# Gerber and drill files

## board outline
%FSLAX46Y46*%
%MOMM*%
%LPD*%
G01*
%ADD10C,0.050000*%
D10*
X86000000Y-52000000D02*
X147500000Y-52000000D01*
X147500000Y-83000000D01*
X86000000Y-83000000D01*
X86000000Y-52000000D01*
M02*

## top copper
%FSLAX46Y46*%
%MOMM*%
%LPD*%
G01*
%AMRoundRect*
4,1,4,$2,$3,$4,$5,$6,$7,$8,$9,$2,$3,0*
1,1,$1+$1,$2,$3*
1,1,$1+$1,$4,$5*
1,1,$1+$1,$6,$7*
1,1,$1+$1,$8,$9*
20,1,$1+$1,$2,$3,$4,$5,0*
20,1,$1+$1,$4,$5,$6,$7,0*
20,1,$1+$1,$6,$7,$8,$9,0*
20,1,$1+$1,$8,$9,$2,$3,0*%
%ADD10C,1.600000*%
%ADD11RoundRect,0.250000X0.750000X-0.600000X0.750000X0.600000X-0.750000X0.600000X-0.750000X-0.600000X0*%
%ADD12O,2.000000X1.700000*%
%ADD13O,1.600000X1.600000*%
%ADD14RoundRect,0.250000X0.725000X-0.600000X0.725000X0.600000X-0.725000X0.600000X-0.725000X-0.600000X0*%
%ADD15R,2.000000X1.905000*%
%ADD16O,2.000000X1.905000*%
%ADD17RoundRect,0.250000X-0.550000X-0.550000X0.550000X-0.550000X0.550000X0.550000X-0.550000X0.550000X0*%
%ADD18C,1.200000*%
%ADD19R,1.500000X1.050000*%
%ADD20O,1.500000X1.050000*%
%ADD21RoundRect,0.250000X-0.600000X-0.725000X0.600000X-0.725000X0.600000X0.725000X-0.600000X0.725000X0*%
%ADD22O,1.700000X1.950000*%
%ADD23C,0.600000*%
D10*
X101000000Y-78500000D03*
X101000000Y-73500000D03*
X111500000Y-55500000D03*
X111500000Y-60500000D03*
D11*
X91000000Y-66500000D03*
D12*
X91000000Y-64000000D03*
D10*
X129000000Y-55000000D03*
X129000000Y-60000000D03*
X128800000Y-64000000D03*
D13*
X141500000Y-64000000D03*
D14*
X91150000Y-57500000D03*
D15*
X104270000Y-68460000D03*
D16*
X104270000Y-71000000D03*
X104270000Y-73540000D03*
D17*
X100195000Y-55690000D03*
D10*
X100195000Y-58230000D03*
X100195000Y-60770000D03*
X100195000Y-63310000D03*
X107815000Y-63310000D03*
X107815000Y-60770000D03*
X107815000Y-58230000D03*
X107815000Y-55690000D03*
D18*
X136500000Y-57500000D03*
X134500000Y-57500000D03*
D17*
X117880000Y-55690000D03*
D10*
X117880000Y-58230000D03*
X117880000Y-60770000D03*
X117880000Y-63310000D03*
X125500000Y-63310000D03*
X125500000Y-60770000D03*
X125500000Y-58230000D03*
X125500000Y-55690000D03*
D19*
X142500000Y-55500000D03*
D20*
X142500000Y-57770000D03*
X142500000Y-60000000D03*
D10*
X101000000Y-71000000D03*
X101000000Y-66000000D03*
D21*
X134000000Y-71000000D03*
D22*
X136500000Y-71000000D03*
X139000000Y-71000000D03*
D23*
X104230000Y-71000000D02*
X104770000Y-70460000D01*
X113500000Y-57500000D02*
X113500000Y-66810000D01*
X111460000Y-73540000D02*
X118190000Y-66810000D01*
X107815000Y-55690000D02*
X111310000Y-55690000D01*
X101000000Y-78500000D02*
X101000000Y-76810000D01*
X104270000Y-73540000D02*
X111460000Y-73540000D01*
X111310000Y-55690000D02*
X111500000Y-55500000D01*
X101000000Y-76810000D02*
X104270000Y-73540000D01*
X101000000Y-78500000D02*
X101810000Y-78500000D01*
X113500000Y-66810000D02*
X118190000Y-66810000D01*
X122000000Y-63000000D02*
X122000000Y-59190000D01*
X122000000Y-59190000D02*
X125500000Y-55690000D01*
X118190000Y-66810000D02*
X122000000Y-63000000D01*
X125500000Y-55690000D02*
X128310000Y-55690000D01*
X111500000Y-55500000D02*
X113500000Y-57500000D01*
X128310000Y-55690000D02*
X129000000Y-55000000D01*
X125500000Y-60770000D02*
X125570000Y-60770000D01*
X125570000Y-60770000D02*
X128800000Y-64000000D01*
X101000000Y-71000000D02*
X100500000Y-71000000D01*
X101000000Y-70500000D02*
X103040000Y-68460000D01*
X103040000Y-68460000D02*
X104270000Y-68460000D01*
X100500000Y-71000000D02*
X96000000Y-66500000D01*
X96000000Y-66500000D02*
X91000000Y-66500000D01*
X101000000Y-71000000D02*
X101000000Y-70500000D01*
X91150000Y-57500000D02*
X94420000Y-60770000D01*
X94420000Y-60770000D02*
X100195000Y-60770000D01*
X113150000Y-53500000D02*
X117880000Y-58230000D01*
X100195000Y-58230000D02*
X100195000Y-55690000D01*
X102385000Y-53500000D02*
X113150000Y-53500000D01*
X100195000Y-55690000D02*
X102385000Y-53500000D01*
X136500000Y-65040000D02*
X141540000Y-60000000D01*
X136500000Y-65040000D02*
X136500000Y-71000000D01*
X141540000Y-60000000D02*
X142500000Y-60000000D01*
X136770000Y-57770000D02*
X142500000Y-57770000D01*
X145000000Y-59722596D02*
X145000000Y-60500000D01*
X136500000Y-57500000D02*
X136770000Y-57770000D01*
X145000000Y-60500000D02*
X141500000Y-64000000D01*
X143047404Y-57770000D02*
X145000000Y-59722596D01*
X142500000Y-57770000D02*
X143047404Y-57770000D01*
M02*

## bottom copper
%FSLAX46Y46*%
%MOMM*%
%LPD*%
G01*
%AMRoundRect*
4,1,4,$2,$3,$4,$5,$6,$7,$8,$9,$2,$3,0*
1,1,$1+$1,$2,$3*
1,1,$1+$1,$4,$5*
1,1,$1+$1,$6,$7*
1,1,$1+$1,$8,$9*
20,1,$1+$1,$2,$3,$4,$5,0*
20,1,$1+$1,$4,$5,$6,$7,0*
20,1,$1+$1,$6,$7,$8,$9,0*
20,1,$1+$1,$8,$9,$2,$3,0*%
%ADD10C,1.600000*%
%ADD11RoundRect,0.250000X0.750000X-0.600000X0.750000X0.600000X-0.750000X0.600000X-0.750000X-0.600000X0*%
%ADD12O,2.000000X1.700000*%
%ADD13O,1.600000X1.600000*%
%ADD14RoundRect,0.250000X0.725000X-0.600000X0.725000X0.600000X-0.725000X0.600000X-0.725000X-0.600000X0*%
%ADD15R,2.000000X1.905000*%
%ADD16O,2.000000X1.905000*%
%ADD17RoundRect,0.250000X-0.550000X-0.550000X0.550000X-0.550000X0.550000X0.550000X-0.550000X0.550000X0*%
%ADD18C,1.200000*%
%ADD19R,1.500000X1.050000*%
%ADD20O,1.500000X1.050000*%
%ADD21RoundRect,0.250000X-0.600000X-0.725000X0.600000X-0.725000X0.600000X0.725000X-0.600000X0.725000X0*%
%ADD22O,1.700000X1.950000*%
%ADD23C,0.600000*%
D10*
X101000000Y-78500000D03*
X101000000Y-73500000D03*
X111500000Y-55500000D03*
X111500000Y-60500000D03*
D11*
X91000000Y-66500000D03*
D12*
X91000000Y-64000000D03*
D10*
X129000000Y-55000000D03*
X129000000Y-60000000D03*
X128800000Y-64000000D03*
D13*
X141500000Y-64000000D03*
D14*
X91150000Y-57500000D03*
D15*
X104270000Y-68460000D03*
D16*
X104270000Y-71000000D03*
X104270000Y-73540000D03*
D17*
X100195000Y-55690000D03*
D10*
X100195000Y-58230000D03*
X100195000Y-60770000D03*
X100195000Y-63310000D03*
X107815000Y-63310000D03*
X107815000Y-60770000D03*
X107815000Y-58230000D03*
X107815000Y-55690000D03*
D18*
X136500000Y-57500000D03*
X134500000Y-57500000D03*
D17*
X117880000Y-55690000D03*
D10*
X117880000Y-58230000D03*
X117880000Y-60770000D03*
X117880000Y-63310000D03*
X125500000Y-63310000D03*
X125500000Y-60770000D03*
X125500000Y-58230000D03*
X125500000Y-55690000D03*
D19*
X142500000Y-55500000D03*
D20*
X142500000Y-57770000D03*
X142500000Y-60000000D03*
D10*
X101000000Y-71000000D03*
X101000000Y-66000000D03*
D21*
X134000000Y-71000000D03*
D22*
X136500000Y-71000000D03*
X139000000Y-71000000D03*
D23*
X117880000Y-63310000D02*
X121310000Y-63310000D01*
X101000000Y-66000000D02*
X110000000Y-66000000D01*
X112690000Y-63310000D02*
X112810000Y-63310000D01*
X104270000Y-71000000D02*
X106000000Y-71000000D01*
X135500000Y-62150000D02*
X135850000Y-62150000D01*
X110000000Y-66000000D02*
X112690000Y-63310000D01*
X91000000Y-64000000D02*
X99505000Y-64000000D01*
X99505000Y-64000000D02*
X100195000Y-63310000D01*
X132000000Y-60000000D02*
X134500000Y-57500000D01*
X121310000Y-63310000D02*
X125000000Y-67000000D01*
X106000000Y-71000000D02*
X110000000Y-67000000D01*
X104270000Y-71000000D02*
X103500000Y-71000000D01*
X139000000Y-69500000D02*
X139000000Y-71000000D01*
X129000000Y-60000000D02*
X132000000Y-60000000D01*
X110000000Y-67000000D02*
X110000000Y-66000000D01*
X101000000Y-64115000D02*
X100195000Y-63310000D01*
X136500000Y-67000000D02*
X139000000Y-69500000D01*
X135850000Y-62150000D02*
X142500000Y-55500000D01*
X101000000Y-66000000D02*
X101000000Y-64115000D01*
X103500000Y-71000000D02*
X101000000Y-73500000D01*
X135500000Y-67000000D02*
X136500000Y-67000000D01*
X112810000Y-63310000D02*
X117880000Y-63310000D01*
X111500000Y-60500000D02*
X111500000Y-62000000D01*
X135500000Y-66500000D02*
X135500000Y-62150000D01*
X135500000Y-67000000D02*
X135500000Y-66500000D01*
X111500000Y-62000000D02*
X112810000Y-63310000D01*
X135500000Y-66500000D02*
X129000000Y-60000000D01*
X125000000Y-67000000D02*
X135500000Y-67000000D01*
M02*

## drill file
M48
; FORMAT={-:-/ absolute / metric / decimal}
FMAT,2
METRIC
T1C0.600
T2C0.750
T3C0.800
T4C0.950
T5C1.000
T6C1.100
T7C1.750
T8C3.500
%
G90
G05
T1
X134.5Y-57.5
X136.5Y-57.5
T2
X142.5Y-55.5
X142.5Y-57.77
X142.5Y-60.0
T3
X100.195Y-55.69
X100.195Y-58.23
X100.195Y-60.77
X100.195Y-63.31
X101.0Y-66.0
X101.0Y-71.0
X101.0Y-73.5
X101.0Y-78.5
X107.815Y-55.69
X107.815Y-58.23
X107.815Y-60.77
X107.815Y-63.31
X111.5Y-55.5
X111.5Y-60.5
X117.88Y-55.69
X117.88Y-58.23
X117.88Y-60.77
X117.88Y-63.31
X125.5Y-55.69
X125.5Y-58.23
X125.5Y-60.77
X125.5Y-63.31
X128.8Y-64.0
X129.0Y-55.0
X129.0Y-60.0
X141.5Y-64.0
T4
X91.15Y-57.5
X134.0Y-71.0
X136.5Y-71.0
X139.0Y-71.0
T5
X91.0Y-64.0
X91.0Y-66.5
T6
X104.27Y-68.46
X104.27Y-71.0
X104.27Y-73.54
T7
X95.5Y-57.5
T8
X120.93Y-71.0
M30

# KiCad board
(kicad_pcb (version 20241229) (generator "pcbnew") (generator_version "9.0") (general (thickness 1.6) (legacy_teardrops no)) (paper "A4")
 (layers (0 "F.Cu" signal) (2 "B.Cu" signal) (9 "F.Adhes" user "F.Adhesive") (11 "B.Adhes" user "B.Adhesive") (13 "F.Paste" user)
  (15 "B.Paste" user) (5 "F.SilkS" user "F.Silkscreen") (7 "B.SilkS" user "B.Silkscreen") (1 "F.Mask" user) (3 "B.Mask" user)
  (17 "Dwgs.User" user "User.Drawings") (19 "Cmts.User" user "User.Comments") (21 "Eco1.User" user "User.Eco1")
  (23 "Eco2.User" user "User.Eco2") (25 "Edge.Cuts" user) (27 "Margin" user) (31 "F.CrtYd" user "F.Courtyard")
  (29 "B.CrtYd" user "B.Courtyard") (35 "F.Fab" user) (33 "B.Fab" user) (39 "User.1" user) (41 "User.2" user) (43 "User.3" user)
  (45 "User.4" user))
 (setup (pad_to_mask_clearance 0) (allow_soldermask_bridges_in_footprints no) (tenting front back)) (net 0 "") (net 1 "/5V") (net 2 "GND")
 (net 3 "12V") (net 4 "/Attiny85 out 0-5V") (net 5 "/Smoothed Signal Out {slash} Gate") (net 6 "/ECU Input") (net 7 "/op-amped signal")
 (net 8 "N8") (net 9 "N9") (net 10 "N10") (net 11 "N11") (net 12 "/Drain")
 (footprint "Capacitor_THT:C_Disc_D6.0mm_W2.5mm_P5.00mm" (layer "F.Cu") (at 101 78.5 90)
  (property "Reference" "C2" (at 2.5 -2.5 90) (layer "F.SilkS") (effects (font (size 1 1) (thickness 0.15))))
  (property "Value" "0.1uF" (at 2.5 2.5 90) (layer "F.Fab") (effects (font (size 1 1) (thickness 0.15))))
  (pad "1" thru_hole circle (at 0 0 90) (size 1.6 1.6) (drill 0.8) (layers "*.Cu" "*.Mask") (remove_unused_layers no) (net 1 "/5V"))
  (pad "2" thru_hole circle (at 5 0 90) (size 1.6 1.6) (drill 0.8) (layers "*.Cu" "*.Mask") (remove_unused_layers no) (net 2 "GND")))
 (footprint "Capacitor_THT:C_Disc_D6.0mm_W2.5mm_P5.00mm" (layer "F.Cu") (at 111.5 55.5 -90)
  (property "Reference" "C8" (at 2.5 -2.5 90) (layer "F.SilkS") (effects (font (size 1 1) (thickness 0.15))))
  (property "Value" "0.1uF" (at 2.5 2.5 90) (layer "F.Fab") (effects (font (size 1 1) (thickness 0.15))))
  (pad "1" thru_hole circle (at 0 0 270) (size 1.6 1.6) (drill 0.8) (layers "*.Cu" "*.Mask") (remove_unused_layers no) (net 1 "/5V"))
  (pad "2" thru_hole circle (at 5 0 270) (size 1.6 1.6) (drill 0.8) (layers "*.Cu" "*.Mask") (remove_unused_layers no) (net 2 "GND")))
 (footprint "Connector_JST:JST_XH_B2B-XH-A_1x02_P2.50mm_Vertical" (layer "F.Cu") (at 91 66.5 90)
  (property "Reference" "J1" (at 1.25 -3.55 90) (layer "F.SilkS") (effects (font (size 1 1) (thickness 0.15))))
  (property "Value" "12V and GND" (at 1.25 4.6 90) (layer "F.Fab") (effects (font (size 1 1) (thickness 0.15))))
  (pad "1" thru_hole roundrect (at 0 0 90) (size 1.7 2) (drill 1) (layers "*.Cu" "*.Mask") (remove_unused_layers no)
   (roundrect_rratio 0.147059) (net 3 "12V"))
  (pad "2" thru_hole oval (at 2.5 0 90) (size 1.7 2) (drill 1) (layers "*.Cu" "*.Mask") (remove_unused_layers no) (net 2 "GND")))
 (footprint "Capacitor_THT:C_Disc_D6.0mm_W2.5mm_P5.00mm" (layer "F.Cu") (at 129 55 -90)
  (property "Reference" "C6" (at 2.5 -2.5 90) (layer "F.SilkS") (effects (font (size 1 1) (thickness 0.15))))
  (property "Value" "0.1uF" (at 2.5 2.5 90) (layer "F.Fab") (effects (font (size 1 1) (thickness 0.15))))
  (pad "1" thru_hole circle (at 0 0 270) (size 1.6 1.6) (drill 0.8) (layers "*.Cu" "*.Mask") (remove_unused_layers no) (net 1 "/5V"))
  (pad "2" thru_hole circle (at 5 0 270) (size 1.6 1.6) (drill 0.8) (layers "*.Cu" "*.Mask") (remove_unused_layers no) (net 2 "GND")))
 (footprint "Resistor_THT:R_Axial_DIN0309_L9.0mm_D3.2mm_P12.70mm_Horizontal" (layer "F.Cu") (at 128.8 64)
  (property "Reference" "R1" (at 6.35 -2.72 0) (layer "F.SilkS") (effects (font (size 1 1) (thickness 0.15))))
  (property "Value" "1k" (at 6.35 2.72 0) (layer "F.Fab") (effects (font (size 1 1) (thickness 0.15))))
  (pad "1" thru_hole circle (at 0 0) (size 1.6 1.6) (drill 0.8) (layers "*.Cu" "*.Mask") (remove_unused_layers no)
   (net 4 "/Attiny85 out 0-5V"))
  (pad "2" thru_hole oval (at 12.7 0) (size 1.6 1.6) (drill 0.8) (layers "*.Cu" "*.Mask") (remove_unused_layers no)
   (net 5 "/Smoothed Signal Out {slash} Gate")))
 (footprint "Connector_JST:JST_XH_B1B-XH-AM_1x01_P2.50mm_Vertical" (layer "F.Cu") (at 91.15 57.5 90)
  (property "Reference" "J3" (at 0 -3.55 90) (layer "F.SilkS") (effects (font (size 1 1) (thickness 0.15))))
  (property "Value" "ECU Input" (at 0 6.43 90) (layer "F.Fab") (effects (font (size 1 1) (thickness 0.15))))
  (pad "" np_thru_hole circle (at 0 4.35 90) (size 1.75 1.75) (drill 1.75) (layers "*.Cu" "*.Mask"))
  (pad "1" thru_hole roundrect (at 0 0 90) (size 1.7 1.95) (drill 0.95) (layers "*.Cu" "*.Mask") (remove_unused_layers no)
   (roundrect_rratio 0.147059) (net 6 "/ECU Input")))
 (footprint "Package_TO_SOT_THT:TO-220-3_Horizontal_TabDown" (layer "F.Cu") (at 104.27 68.46 -90)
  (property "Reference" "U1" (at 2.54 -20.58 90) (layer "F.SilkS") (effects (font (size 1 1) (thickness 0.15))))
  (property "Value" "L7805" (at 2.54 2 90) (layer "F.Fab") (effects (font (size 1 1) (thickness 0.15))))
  (pad "" np_thru_hole circle (at 2.54 -16.66 270) (size 3.5 3.5) (drill 3.5) (layers "*.Cu" "*.Mask"))
  (pad "1" thru_hole rect (at 0 0 270) (size 1.905 2) (drill 1.1) (layers "*.Cu" "*.Mask") (remove_unused_layers no) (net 3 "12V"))
  (pad "2" thru_hole oval (at 2.54 0 270) (size 1.905 2) (drill 1.1) (layers "*.Cu" "*.Mask") (remove_unused_layers no) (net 2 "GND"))
  (pad "3" thru_hole oval (at 5.08 0 270) (size 1.905 2) (drill 1.1) (layers "*.Cu" "*.Mask") (remove_unused_layers no) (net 1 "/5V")))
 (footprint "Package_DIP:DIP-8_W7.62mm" (layer "F.Cu") (at 100.195 55.69)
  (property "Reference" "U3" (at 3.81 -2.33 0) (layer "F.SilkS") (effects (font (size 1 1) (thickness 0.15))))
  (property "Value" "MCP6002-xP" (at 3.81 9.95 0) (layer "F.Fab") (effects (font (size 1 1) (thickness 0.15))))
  (pad "1" thru_hole roundrect (at 0 0) (size 1.6 1.6) (drill 0.8) (layers "*.Cu" "*.Mask") (remove_unused_layers no)
   (roundrect_rratio 0.15625) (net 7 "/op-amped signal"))
  (pad "2" thru_hole circle (at 0 2.54) (size 1.6 1.6) (drill 0.8) (layers "*.Cu" "*.Mask") (remove_unused_layers no)
   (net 7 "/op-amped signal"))
  (pad "3" thru_hole circle (at 0 5.08) (size 1.6 1.6) (drill 0.8) (layers "*.Cu" "*.Mask") (remove_unused_layers no) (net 6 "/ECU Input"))
  (pad "4" thru_hole circle (at 0 7.62) (size 1.6 1.6) (drill 0.8) (layers "*.Cu" "*.Mask") (remove_unused_layers no) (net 2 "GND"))
  (pad "5" thru_hole circle (at 7.62 7.62) (size 1.6 1.6) (drill 0.8) (layers "*.Cu" "*.Mask") (remove_unused_layers no))
  (pad "6" thru_hole circle (at 7.62 5.08) (size 1.6 1.6) (drill 0.8) (layers "*.Cu" "*.Mask") (remove_unused_layers no))
  (pad "7" thru_hole circle (at 7.62 2.54) (size 1.6 1.6) (drill 0.8) (layers "*.Cu" "*.Mask") (remove_unused_layers no))
  (pad "8" thru_hole circle (at 7.62 0) (size 1.6 1.6) (drill 0.8) (layers "*.Cu" "*.Mask") (remove_unused_layers no) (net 1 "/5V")))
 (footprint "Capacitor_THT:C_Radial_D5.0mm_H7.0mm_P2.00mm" (layer "F.Cu") (at 136.5 57.5 180)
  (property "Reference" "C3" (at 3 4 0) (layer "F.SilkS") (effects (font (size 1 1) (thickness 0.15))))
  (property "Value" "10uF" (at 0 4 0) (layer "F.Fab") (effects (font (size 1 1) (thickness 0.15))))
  (pad "1" thru_hole circle (at 0 0 180) (size 1.2 1.2) (drill 0.6) (layers "*.Cu" "*.Mask") (remove_unused_layers no)
   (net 5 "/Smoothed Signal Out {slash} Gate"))
  (pad "2" thru_hole circle (at 2 0 180) (size 1.2 1.2) (drill 0.6) (layers "*.Cu" "*.Mask") (remove_unused_layers no) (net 2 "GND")))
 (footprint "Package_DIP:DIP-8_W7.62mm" (layer "F.Cu") (at 117.88 55.69)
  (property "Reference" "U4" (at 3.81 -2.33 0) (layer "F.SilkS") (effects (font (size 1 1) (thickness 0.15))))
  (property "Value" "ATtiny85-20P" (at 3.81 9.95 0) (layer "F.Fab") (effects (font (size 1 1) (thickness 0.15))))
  (pad "1" thru_hole roundrect (at 0 0) (size 1.6 1.6) (drill 0.8) (layers "*.Cu" "*.Mask") (remove_unused_layers no)
   (roundrect_rratio 0.15625) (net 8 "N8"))
  (pad "2" thru_hole circle (at 0 2.54) (size 1.6 1.6) (drill 0.8) (layers "*.Cu" "*.Mask") (remove_unused_layers no)
   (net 7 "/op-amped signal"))
  (pad "3" thru_hole circle (at 0 5.08) (size 1.6 1.6) (drill 0.8) (layers "*.Cu" "*.Mask") (remove_unused_layers no) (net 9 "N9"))
  (pad "4" thru_hole circle (at 0 7.62) (size 1.6 1.6) (drill 0.8) (layers "*.Cu" "*.Mask") (remove_unused_layers no) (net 2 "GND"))
  (pad "5" thru_hole circle (at 7.62 7.62) (size 1.6 1.6) (drill 0.8) (layers "*.Cu" "*.Mask") (remove_unused_layers no) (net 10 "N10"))
  (pad "6" thru_hole circle (at 7.62 5.08) (size 1.6 1.6) (drill 0.8) (layers "*.Cu" "*.Mask") (remove_unused_layers no)
   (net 4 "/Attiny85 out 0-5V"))
  (pad "7" thru_hole circle (at 7.62 2.54) (size 1.6 1.6) (drill 0.8) (layers "*.Cu" "*.Mask") (remove_unused_layers no) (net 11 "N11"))
  (pad "8" thru_hole circle (at 7.62 0) (size 1.6 1.6) (drill 0.8) (layers "*.Cu" "*.Mask") (remove_unused_layers no) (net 1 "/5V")))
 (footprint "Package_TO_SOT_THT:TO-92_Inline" (layer "F.Cu") (at 142.5 56.5 -90)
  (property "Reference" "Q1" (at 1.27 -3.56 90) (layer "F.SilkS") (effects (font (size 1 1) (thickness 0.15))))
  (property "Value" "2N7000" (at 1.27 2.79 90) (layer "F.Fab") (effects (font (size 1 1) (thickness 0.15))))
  (pad "1" thru_hole rect (at -1 0 270) (size 1.05 1.5) (drill 0.75) (layers "*.Cu" "*.Mask") (remove_unused_layers no) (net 2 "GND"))
  (pad "2" thru_hole oval (at 1.27 0 270) (size 1.05 1.5) (drill 0.75) (layers "*.Cu" "*.Mask") (remove_unused_layers no)
   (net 5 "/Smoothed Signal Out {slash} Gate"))
  (pad "3" thru_hole oval (at 3.5 0 270) (size 1.05 1.5) (drill 0.75) (layers "*.Cu" "*.Mask") (remove_unused_layers no) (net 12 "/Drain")))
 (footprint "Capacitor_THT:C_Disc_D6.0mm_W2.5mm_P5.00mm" (layer "F.Cu") (at 101 71 90)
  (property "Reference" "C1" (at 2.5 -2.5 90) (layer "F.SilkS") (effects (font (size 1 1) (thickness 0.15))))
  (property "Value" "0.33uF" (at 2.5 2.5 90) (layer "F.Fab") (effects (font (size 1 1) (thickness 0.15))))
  (pad "1" thru_hole circle (at 0 0 90) (size 1.6 1.6) (drill 0.8) (layers "*.Cu" "*.Mask") (remove_unused_layers no) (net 3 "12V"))
  (pad "2" thru_hole circle (at 5 0 90) (size 1.6 1.6) (drill 0.8) (layers "*.Cu" "*.Mask") (remove_unused_layers no) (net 2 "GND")))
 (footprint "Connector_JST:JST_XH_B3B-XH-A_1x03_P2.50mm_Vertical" (layer "F.Cu") (at 134 71)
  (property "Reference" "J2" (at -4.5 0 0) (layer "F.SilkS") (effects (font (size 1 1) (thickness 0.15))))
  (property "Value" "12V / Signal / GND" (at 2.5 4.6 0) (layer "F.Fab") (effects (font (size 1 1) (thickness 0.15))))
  (pad "1" thru_hole roundrect (at 0 0) (size 1.7 1.95) (drill 0.95) (layers "*.Cu" "*.Mask") (remove_unused_layers no)
   (roundrect_rratio 0.147059) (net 3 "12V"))
  (pad "2" thru_hole oval (at 2.5 0) (size 1.7 1.95) (drill 0.95) (layers "*.Cu" "*.Mask") (remove_unused_layers no) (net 12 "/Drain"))
  (pad "3" thru_hole oval (at 5 0) (size 1.7 1.95) (drill 0.95) (layers "*.Cu" "*.Mask") (remove_unused_layers no) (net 2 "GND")))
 (gr_rect (start 86 52) (end 147.5 83) (stroke (width 0.05) (type default)) (fill no) (layer "Edge.Cuts"))
 (segment (start 104.23 71) (end 104.77 70.46) (width 0.6) (layer "F.Cu") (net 2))
 (segment (start 117.88 63.31) (end 121.31 63.31) (width 0.6) (layer "B.Cu") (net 2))
 (segment (start 101 66) (end 110 66) (width 0.6) (layer "B.Cu") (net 2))
 (segment (start 112.69 63.31) (end 112.81 63.31) (width 0.6) (layer "B.Cu") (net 2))
 (segment (start 104.27 71) (end 106 71) (width 0.6) (layer "B.Cu") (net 2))
 (segment (start 135.5 62.15) (end 135.85 62.15) (width 0.6) (layer "B.Cu") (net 2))
 (segment (start 110 66) (end 112.69 63.31) (width 0.6) (layer "B.Cu") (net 2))
 (segment (start 91 64) (end 99.505 64) (width 0.6) (layer "B.Cu") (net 2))
 (segment (start 99.505 64) (end 100.195 63.31) (width 0.6) (layer "B.Cu") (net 2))
 (segment (start 132 60) (end 134.5 57.5) (width 0.6) (layer "B.Cu") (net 2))
 (segment (start 121.31 63.31) (end 125 67) (width 0.6) (layer "B.Cu") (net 2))
 (segment (start 106 71) (end 110 67) (width 0.6) (layer "B.Cu") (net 2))
 (segment (start 104.27 71) (end 103.5 71) (width 0.6) (layer "B.Cu") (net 2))
 (segment (start 139 69.5) (end 139 71) (width 0.6) (layer "B.Cu") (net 2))
 (segment (start 129 60) (end 132 60) (width 0.6) (layer "B.Cu") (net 2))
 (segment (start 110 67) (end 110 66) (width 0.6) (layer "B.Cu") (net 2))
 (segment (start 101 64.115) (end 100.195 63.31) (width 0.6) (layer "B.Cu") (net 2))
 (segment (start 136.5 67) (end 139 69.5) (width 0.6) (layer "B.Cu") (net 2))
 (segment (start 135.85 62.15) (end 142.5 55.5) (width 0.6) (layer "B.Cu") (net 2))
 (segment (start 101 66) (end 101 64.115) (width 0.6) (layer "B.Cu") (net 2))
 (segment (start 103.5 71) (end 101 73.5) (width 0.6) (layer "B.Cu") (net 2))
 (segment (start 135.5 67) (end 136.5 67) (width 0.6) (layer "B.Cu") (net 2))
 (segment (start 112.81 63.31) (end 117.88 63.31) (width 0.6) (layer "B.Cu") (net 2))
 (segment (start 111.5 60.5) (end 111.5 62) (width 0.6) (layer "B.Cu") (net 2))
 (segment (start 135.5 66.5) (end 135.5 62.15) (width 0.6) (layer "B.Cu") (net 2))
 (segment (start 135.5 67) (end 135.5 66.5) (width 0.6) (layer "B.Cu") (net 2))
 (segment (start 111.5 62) (end 112.81 63.31) (width 0.6) (layer "B.Cu") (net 2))
 (segment (start 135.5 66.5) (end 129 60) (width 0.6) (layer "B.Cu") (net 2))
 (segment (start 125 67) (end 135.5 67) (width 0.6) (layer "B.Cu") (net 2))
 (segment (start 113.5 57.5) (end 113.5 66.81) (width 0.6) (layer "F.Cu") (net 1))
 (segment (start 111.46 73.54) (end 118.19 66.81) (width 0.6) (layer "F.Cu") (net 1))
 (segment (start 107.815 55.69) (end 111.31 55.69) (width 0.6) (layer "F.Cu") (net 1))
 (segment (start 101 78.5) (end 101 76.81) (width 0.6) (layer "F.Cu") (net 1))
 (segment (start 104.27 73.54) (end 111.46 73.54) (width 0.6) (layer "F.Cu") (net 1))
 (segment (start 111.31 55.69) (end 111.5 55.5) (width 0.6) (layer "F.Cu") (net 1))
 (segment (start 101 76.81) (end 104.27 73.54) (width 0.6) (layer "F.Cu") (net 1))
 (segment (start 101 78.5) (end 101.81 78.5) (width 0.6) (layer "F.Cu") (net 1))
 (segment (start 113.5 66.81) (end 118.19 66.81) (width 0.6) (layer "F.Cu") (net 1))
 (segment (start 122 63) (end 122 59.19) (width 0.6) (layer "F.Cu") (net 1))
 (segment (start 122 59.19) (end 125.5 55.69) (width 0.6) (layer "F.Cu") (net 1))
 (segment (start 118.19 66.81) (end 122 63) (width 0.6) (layer "F.Cu") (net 1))
 (segment (start 125.5 55.69) (end 128.31 55.69) (width 0.6) (layer "F.Cu") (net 1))
 (segment (start 111.5 55.5) (end 113.5 57.5) (width 0.6) (layer "F.Cu") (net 1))
 (segment (start 128.31 55.69) (end 129 55) (width 0.6) (layer "F.Cu") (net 1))
 (segment (start 125.5 60.77) (end 125.57 60.77) (width 0.6) (layer "F.Cu") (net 4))
 (segment (start 125.57 60.77) (end 128.8 64) (width 0.6) (layer "F.Cu") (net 4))
 (segment (start 101 71) (end 100.5 71) (width 0.6) (layer "F.Cu") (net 3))
 (segment (start 101 70.5) (end 103.04 68.46) (width 0.6) (layer "F.Cu") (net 3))
 (segment (start 103.04 68.46) (end 104.27 68.46) (width 0.6) (layer "F.Cu") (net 3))
 (segment (start 100.5 71) (end 96 66.5) (width 0.6) (layer "F.Cu") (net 3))
 (segment (start 96 66.5) (end 91 66.5) (width 0.6) (layer "F.Cu") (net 3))
 (segment (start 101 71) (end 101 70.5) (width 0.6) (layer "F.Cu") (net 3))
 (segment (start 91.15 57.5) (end 94.42 60.77) (width 0.6) (layer "F.Cu") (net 6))
 (segment (start 94.42 60.77) (end 100.195 60.77) (width 0.6) (layer "F.Cu") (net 6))
 (segment (start 113.15 53.5) (end 117.88 58.23) (width 0.6) (layer "F.Cu") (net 7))
 (segment (start 100.195 58.23) (end 100.195 55.69) (width 0.6) (layer "F.Cu") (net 7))
 (segment (start 102.385 53.5) (end 113.15 53.5) (width 0.6) (layer "F.Cu") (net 7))
 (segment (start 100.195 55.69) (end 102.385 53.5) (width 0.6) (layer "F.Cu") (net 7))
 (segment (start 136.5 65.04) (end 141.54 60) (width 0.6) (layer "F.Cu") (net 12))
 (segment (start 136.5 65.04) (end 136.5 71) (width 0.6) (layer "F.Cu") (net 12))
 (segment (start 141.54 60) (end 142.5 60) (width 0.6) (layer "F.Cu") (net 12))
 (segment (start 136.77 57.77) (end 142.5 57.77) (width 0.6) (layer "F.Cu") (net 5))
 (segment (start 145 59.722596) (end 145 60.5) (width 0.6) (layer "F.Cu") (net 5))
 (segment (start 136.5 57.5) (end 136.77 57.77) (width 0.6) (layer "F.Cu") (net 5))
 (segment (start 145 60.5) (end 141.5 64) (width 0.6) (layer "F.Cu") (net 5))
 (segment (start 143.047404 57.77) (end 145 59.722596) (width 0.6) (layer "F.Cu") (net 5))
 (segment (start 142.5 57.77) (end 143.047404 57.77) (width 0.6) (layer "F.Cu") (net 5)))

